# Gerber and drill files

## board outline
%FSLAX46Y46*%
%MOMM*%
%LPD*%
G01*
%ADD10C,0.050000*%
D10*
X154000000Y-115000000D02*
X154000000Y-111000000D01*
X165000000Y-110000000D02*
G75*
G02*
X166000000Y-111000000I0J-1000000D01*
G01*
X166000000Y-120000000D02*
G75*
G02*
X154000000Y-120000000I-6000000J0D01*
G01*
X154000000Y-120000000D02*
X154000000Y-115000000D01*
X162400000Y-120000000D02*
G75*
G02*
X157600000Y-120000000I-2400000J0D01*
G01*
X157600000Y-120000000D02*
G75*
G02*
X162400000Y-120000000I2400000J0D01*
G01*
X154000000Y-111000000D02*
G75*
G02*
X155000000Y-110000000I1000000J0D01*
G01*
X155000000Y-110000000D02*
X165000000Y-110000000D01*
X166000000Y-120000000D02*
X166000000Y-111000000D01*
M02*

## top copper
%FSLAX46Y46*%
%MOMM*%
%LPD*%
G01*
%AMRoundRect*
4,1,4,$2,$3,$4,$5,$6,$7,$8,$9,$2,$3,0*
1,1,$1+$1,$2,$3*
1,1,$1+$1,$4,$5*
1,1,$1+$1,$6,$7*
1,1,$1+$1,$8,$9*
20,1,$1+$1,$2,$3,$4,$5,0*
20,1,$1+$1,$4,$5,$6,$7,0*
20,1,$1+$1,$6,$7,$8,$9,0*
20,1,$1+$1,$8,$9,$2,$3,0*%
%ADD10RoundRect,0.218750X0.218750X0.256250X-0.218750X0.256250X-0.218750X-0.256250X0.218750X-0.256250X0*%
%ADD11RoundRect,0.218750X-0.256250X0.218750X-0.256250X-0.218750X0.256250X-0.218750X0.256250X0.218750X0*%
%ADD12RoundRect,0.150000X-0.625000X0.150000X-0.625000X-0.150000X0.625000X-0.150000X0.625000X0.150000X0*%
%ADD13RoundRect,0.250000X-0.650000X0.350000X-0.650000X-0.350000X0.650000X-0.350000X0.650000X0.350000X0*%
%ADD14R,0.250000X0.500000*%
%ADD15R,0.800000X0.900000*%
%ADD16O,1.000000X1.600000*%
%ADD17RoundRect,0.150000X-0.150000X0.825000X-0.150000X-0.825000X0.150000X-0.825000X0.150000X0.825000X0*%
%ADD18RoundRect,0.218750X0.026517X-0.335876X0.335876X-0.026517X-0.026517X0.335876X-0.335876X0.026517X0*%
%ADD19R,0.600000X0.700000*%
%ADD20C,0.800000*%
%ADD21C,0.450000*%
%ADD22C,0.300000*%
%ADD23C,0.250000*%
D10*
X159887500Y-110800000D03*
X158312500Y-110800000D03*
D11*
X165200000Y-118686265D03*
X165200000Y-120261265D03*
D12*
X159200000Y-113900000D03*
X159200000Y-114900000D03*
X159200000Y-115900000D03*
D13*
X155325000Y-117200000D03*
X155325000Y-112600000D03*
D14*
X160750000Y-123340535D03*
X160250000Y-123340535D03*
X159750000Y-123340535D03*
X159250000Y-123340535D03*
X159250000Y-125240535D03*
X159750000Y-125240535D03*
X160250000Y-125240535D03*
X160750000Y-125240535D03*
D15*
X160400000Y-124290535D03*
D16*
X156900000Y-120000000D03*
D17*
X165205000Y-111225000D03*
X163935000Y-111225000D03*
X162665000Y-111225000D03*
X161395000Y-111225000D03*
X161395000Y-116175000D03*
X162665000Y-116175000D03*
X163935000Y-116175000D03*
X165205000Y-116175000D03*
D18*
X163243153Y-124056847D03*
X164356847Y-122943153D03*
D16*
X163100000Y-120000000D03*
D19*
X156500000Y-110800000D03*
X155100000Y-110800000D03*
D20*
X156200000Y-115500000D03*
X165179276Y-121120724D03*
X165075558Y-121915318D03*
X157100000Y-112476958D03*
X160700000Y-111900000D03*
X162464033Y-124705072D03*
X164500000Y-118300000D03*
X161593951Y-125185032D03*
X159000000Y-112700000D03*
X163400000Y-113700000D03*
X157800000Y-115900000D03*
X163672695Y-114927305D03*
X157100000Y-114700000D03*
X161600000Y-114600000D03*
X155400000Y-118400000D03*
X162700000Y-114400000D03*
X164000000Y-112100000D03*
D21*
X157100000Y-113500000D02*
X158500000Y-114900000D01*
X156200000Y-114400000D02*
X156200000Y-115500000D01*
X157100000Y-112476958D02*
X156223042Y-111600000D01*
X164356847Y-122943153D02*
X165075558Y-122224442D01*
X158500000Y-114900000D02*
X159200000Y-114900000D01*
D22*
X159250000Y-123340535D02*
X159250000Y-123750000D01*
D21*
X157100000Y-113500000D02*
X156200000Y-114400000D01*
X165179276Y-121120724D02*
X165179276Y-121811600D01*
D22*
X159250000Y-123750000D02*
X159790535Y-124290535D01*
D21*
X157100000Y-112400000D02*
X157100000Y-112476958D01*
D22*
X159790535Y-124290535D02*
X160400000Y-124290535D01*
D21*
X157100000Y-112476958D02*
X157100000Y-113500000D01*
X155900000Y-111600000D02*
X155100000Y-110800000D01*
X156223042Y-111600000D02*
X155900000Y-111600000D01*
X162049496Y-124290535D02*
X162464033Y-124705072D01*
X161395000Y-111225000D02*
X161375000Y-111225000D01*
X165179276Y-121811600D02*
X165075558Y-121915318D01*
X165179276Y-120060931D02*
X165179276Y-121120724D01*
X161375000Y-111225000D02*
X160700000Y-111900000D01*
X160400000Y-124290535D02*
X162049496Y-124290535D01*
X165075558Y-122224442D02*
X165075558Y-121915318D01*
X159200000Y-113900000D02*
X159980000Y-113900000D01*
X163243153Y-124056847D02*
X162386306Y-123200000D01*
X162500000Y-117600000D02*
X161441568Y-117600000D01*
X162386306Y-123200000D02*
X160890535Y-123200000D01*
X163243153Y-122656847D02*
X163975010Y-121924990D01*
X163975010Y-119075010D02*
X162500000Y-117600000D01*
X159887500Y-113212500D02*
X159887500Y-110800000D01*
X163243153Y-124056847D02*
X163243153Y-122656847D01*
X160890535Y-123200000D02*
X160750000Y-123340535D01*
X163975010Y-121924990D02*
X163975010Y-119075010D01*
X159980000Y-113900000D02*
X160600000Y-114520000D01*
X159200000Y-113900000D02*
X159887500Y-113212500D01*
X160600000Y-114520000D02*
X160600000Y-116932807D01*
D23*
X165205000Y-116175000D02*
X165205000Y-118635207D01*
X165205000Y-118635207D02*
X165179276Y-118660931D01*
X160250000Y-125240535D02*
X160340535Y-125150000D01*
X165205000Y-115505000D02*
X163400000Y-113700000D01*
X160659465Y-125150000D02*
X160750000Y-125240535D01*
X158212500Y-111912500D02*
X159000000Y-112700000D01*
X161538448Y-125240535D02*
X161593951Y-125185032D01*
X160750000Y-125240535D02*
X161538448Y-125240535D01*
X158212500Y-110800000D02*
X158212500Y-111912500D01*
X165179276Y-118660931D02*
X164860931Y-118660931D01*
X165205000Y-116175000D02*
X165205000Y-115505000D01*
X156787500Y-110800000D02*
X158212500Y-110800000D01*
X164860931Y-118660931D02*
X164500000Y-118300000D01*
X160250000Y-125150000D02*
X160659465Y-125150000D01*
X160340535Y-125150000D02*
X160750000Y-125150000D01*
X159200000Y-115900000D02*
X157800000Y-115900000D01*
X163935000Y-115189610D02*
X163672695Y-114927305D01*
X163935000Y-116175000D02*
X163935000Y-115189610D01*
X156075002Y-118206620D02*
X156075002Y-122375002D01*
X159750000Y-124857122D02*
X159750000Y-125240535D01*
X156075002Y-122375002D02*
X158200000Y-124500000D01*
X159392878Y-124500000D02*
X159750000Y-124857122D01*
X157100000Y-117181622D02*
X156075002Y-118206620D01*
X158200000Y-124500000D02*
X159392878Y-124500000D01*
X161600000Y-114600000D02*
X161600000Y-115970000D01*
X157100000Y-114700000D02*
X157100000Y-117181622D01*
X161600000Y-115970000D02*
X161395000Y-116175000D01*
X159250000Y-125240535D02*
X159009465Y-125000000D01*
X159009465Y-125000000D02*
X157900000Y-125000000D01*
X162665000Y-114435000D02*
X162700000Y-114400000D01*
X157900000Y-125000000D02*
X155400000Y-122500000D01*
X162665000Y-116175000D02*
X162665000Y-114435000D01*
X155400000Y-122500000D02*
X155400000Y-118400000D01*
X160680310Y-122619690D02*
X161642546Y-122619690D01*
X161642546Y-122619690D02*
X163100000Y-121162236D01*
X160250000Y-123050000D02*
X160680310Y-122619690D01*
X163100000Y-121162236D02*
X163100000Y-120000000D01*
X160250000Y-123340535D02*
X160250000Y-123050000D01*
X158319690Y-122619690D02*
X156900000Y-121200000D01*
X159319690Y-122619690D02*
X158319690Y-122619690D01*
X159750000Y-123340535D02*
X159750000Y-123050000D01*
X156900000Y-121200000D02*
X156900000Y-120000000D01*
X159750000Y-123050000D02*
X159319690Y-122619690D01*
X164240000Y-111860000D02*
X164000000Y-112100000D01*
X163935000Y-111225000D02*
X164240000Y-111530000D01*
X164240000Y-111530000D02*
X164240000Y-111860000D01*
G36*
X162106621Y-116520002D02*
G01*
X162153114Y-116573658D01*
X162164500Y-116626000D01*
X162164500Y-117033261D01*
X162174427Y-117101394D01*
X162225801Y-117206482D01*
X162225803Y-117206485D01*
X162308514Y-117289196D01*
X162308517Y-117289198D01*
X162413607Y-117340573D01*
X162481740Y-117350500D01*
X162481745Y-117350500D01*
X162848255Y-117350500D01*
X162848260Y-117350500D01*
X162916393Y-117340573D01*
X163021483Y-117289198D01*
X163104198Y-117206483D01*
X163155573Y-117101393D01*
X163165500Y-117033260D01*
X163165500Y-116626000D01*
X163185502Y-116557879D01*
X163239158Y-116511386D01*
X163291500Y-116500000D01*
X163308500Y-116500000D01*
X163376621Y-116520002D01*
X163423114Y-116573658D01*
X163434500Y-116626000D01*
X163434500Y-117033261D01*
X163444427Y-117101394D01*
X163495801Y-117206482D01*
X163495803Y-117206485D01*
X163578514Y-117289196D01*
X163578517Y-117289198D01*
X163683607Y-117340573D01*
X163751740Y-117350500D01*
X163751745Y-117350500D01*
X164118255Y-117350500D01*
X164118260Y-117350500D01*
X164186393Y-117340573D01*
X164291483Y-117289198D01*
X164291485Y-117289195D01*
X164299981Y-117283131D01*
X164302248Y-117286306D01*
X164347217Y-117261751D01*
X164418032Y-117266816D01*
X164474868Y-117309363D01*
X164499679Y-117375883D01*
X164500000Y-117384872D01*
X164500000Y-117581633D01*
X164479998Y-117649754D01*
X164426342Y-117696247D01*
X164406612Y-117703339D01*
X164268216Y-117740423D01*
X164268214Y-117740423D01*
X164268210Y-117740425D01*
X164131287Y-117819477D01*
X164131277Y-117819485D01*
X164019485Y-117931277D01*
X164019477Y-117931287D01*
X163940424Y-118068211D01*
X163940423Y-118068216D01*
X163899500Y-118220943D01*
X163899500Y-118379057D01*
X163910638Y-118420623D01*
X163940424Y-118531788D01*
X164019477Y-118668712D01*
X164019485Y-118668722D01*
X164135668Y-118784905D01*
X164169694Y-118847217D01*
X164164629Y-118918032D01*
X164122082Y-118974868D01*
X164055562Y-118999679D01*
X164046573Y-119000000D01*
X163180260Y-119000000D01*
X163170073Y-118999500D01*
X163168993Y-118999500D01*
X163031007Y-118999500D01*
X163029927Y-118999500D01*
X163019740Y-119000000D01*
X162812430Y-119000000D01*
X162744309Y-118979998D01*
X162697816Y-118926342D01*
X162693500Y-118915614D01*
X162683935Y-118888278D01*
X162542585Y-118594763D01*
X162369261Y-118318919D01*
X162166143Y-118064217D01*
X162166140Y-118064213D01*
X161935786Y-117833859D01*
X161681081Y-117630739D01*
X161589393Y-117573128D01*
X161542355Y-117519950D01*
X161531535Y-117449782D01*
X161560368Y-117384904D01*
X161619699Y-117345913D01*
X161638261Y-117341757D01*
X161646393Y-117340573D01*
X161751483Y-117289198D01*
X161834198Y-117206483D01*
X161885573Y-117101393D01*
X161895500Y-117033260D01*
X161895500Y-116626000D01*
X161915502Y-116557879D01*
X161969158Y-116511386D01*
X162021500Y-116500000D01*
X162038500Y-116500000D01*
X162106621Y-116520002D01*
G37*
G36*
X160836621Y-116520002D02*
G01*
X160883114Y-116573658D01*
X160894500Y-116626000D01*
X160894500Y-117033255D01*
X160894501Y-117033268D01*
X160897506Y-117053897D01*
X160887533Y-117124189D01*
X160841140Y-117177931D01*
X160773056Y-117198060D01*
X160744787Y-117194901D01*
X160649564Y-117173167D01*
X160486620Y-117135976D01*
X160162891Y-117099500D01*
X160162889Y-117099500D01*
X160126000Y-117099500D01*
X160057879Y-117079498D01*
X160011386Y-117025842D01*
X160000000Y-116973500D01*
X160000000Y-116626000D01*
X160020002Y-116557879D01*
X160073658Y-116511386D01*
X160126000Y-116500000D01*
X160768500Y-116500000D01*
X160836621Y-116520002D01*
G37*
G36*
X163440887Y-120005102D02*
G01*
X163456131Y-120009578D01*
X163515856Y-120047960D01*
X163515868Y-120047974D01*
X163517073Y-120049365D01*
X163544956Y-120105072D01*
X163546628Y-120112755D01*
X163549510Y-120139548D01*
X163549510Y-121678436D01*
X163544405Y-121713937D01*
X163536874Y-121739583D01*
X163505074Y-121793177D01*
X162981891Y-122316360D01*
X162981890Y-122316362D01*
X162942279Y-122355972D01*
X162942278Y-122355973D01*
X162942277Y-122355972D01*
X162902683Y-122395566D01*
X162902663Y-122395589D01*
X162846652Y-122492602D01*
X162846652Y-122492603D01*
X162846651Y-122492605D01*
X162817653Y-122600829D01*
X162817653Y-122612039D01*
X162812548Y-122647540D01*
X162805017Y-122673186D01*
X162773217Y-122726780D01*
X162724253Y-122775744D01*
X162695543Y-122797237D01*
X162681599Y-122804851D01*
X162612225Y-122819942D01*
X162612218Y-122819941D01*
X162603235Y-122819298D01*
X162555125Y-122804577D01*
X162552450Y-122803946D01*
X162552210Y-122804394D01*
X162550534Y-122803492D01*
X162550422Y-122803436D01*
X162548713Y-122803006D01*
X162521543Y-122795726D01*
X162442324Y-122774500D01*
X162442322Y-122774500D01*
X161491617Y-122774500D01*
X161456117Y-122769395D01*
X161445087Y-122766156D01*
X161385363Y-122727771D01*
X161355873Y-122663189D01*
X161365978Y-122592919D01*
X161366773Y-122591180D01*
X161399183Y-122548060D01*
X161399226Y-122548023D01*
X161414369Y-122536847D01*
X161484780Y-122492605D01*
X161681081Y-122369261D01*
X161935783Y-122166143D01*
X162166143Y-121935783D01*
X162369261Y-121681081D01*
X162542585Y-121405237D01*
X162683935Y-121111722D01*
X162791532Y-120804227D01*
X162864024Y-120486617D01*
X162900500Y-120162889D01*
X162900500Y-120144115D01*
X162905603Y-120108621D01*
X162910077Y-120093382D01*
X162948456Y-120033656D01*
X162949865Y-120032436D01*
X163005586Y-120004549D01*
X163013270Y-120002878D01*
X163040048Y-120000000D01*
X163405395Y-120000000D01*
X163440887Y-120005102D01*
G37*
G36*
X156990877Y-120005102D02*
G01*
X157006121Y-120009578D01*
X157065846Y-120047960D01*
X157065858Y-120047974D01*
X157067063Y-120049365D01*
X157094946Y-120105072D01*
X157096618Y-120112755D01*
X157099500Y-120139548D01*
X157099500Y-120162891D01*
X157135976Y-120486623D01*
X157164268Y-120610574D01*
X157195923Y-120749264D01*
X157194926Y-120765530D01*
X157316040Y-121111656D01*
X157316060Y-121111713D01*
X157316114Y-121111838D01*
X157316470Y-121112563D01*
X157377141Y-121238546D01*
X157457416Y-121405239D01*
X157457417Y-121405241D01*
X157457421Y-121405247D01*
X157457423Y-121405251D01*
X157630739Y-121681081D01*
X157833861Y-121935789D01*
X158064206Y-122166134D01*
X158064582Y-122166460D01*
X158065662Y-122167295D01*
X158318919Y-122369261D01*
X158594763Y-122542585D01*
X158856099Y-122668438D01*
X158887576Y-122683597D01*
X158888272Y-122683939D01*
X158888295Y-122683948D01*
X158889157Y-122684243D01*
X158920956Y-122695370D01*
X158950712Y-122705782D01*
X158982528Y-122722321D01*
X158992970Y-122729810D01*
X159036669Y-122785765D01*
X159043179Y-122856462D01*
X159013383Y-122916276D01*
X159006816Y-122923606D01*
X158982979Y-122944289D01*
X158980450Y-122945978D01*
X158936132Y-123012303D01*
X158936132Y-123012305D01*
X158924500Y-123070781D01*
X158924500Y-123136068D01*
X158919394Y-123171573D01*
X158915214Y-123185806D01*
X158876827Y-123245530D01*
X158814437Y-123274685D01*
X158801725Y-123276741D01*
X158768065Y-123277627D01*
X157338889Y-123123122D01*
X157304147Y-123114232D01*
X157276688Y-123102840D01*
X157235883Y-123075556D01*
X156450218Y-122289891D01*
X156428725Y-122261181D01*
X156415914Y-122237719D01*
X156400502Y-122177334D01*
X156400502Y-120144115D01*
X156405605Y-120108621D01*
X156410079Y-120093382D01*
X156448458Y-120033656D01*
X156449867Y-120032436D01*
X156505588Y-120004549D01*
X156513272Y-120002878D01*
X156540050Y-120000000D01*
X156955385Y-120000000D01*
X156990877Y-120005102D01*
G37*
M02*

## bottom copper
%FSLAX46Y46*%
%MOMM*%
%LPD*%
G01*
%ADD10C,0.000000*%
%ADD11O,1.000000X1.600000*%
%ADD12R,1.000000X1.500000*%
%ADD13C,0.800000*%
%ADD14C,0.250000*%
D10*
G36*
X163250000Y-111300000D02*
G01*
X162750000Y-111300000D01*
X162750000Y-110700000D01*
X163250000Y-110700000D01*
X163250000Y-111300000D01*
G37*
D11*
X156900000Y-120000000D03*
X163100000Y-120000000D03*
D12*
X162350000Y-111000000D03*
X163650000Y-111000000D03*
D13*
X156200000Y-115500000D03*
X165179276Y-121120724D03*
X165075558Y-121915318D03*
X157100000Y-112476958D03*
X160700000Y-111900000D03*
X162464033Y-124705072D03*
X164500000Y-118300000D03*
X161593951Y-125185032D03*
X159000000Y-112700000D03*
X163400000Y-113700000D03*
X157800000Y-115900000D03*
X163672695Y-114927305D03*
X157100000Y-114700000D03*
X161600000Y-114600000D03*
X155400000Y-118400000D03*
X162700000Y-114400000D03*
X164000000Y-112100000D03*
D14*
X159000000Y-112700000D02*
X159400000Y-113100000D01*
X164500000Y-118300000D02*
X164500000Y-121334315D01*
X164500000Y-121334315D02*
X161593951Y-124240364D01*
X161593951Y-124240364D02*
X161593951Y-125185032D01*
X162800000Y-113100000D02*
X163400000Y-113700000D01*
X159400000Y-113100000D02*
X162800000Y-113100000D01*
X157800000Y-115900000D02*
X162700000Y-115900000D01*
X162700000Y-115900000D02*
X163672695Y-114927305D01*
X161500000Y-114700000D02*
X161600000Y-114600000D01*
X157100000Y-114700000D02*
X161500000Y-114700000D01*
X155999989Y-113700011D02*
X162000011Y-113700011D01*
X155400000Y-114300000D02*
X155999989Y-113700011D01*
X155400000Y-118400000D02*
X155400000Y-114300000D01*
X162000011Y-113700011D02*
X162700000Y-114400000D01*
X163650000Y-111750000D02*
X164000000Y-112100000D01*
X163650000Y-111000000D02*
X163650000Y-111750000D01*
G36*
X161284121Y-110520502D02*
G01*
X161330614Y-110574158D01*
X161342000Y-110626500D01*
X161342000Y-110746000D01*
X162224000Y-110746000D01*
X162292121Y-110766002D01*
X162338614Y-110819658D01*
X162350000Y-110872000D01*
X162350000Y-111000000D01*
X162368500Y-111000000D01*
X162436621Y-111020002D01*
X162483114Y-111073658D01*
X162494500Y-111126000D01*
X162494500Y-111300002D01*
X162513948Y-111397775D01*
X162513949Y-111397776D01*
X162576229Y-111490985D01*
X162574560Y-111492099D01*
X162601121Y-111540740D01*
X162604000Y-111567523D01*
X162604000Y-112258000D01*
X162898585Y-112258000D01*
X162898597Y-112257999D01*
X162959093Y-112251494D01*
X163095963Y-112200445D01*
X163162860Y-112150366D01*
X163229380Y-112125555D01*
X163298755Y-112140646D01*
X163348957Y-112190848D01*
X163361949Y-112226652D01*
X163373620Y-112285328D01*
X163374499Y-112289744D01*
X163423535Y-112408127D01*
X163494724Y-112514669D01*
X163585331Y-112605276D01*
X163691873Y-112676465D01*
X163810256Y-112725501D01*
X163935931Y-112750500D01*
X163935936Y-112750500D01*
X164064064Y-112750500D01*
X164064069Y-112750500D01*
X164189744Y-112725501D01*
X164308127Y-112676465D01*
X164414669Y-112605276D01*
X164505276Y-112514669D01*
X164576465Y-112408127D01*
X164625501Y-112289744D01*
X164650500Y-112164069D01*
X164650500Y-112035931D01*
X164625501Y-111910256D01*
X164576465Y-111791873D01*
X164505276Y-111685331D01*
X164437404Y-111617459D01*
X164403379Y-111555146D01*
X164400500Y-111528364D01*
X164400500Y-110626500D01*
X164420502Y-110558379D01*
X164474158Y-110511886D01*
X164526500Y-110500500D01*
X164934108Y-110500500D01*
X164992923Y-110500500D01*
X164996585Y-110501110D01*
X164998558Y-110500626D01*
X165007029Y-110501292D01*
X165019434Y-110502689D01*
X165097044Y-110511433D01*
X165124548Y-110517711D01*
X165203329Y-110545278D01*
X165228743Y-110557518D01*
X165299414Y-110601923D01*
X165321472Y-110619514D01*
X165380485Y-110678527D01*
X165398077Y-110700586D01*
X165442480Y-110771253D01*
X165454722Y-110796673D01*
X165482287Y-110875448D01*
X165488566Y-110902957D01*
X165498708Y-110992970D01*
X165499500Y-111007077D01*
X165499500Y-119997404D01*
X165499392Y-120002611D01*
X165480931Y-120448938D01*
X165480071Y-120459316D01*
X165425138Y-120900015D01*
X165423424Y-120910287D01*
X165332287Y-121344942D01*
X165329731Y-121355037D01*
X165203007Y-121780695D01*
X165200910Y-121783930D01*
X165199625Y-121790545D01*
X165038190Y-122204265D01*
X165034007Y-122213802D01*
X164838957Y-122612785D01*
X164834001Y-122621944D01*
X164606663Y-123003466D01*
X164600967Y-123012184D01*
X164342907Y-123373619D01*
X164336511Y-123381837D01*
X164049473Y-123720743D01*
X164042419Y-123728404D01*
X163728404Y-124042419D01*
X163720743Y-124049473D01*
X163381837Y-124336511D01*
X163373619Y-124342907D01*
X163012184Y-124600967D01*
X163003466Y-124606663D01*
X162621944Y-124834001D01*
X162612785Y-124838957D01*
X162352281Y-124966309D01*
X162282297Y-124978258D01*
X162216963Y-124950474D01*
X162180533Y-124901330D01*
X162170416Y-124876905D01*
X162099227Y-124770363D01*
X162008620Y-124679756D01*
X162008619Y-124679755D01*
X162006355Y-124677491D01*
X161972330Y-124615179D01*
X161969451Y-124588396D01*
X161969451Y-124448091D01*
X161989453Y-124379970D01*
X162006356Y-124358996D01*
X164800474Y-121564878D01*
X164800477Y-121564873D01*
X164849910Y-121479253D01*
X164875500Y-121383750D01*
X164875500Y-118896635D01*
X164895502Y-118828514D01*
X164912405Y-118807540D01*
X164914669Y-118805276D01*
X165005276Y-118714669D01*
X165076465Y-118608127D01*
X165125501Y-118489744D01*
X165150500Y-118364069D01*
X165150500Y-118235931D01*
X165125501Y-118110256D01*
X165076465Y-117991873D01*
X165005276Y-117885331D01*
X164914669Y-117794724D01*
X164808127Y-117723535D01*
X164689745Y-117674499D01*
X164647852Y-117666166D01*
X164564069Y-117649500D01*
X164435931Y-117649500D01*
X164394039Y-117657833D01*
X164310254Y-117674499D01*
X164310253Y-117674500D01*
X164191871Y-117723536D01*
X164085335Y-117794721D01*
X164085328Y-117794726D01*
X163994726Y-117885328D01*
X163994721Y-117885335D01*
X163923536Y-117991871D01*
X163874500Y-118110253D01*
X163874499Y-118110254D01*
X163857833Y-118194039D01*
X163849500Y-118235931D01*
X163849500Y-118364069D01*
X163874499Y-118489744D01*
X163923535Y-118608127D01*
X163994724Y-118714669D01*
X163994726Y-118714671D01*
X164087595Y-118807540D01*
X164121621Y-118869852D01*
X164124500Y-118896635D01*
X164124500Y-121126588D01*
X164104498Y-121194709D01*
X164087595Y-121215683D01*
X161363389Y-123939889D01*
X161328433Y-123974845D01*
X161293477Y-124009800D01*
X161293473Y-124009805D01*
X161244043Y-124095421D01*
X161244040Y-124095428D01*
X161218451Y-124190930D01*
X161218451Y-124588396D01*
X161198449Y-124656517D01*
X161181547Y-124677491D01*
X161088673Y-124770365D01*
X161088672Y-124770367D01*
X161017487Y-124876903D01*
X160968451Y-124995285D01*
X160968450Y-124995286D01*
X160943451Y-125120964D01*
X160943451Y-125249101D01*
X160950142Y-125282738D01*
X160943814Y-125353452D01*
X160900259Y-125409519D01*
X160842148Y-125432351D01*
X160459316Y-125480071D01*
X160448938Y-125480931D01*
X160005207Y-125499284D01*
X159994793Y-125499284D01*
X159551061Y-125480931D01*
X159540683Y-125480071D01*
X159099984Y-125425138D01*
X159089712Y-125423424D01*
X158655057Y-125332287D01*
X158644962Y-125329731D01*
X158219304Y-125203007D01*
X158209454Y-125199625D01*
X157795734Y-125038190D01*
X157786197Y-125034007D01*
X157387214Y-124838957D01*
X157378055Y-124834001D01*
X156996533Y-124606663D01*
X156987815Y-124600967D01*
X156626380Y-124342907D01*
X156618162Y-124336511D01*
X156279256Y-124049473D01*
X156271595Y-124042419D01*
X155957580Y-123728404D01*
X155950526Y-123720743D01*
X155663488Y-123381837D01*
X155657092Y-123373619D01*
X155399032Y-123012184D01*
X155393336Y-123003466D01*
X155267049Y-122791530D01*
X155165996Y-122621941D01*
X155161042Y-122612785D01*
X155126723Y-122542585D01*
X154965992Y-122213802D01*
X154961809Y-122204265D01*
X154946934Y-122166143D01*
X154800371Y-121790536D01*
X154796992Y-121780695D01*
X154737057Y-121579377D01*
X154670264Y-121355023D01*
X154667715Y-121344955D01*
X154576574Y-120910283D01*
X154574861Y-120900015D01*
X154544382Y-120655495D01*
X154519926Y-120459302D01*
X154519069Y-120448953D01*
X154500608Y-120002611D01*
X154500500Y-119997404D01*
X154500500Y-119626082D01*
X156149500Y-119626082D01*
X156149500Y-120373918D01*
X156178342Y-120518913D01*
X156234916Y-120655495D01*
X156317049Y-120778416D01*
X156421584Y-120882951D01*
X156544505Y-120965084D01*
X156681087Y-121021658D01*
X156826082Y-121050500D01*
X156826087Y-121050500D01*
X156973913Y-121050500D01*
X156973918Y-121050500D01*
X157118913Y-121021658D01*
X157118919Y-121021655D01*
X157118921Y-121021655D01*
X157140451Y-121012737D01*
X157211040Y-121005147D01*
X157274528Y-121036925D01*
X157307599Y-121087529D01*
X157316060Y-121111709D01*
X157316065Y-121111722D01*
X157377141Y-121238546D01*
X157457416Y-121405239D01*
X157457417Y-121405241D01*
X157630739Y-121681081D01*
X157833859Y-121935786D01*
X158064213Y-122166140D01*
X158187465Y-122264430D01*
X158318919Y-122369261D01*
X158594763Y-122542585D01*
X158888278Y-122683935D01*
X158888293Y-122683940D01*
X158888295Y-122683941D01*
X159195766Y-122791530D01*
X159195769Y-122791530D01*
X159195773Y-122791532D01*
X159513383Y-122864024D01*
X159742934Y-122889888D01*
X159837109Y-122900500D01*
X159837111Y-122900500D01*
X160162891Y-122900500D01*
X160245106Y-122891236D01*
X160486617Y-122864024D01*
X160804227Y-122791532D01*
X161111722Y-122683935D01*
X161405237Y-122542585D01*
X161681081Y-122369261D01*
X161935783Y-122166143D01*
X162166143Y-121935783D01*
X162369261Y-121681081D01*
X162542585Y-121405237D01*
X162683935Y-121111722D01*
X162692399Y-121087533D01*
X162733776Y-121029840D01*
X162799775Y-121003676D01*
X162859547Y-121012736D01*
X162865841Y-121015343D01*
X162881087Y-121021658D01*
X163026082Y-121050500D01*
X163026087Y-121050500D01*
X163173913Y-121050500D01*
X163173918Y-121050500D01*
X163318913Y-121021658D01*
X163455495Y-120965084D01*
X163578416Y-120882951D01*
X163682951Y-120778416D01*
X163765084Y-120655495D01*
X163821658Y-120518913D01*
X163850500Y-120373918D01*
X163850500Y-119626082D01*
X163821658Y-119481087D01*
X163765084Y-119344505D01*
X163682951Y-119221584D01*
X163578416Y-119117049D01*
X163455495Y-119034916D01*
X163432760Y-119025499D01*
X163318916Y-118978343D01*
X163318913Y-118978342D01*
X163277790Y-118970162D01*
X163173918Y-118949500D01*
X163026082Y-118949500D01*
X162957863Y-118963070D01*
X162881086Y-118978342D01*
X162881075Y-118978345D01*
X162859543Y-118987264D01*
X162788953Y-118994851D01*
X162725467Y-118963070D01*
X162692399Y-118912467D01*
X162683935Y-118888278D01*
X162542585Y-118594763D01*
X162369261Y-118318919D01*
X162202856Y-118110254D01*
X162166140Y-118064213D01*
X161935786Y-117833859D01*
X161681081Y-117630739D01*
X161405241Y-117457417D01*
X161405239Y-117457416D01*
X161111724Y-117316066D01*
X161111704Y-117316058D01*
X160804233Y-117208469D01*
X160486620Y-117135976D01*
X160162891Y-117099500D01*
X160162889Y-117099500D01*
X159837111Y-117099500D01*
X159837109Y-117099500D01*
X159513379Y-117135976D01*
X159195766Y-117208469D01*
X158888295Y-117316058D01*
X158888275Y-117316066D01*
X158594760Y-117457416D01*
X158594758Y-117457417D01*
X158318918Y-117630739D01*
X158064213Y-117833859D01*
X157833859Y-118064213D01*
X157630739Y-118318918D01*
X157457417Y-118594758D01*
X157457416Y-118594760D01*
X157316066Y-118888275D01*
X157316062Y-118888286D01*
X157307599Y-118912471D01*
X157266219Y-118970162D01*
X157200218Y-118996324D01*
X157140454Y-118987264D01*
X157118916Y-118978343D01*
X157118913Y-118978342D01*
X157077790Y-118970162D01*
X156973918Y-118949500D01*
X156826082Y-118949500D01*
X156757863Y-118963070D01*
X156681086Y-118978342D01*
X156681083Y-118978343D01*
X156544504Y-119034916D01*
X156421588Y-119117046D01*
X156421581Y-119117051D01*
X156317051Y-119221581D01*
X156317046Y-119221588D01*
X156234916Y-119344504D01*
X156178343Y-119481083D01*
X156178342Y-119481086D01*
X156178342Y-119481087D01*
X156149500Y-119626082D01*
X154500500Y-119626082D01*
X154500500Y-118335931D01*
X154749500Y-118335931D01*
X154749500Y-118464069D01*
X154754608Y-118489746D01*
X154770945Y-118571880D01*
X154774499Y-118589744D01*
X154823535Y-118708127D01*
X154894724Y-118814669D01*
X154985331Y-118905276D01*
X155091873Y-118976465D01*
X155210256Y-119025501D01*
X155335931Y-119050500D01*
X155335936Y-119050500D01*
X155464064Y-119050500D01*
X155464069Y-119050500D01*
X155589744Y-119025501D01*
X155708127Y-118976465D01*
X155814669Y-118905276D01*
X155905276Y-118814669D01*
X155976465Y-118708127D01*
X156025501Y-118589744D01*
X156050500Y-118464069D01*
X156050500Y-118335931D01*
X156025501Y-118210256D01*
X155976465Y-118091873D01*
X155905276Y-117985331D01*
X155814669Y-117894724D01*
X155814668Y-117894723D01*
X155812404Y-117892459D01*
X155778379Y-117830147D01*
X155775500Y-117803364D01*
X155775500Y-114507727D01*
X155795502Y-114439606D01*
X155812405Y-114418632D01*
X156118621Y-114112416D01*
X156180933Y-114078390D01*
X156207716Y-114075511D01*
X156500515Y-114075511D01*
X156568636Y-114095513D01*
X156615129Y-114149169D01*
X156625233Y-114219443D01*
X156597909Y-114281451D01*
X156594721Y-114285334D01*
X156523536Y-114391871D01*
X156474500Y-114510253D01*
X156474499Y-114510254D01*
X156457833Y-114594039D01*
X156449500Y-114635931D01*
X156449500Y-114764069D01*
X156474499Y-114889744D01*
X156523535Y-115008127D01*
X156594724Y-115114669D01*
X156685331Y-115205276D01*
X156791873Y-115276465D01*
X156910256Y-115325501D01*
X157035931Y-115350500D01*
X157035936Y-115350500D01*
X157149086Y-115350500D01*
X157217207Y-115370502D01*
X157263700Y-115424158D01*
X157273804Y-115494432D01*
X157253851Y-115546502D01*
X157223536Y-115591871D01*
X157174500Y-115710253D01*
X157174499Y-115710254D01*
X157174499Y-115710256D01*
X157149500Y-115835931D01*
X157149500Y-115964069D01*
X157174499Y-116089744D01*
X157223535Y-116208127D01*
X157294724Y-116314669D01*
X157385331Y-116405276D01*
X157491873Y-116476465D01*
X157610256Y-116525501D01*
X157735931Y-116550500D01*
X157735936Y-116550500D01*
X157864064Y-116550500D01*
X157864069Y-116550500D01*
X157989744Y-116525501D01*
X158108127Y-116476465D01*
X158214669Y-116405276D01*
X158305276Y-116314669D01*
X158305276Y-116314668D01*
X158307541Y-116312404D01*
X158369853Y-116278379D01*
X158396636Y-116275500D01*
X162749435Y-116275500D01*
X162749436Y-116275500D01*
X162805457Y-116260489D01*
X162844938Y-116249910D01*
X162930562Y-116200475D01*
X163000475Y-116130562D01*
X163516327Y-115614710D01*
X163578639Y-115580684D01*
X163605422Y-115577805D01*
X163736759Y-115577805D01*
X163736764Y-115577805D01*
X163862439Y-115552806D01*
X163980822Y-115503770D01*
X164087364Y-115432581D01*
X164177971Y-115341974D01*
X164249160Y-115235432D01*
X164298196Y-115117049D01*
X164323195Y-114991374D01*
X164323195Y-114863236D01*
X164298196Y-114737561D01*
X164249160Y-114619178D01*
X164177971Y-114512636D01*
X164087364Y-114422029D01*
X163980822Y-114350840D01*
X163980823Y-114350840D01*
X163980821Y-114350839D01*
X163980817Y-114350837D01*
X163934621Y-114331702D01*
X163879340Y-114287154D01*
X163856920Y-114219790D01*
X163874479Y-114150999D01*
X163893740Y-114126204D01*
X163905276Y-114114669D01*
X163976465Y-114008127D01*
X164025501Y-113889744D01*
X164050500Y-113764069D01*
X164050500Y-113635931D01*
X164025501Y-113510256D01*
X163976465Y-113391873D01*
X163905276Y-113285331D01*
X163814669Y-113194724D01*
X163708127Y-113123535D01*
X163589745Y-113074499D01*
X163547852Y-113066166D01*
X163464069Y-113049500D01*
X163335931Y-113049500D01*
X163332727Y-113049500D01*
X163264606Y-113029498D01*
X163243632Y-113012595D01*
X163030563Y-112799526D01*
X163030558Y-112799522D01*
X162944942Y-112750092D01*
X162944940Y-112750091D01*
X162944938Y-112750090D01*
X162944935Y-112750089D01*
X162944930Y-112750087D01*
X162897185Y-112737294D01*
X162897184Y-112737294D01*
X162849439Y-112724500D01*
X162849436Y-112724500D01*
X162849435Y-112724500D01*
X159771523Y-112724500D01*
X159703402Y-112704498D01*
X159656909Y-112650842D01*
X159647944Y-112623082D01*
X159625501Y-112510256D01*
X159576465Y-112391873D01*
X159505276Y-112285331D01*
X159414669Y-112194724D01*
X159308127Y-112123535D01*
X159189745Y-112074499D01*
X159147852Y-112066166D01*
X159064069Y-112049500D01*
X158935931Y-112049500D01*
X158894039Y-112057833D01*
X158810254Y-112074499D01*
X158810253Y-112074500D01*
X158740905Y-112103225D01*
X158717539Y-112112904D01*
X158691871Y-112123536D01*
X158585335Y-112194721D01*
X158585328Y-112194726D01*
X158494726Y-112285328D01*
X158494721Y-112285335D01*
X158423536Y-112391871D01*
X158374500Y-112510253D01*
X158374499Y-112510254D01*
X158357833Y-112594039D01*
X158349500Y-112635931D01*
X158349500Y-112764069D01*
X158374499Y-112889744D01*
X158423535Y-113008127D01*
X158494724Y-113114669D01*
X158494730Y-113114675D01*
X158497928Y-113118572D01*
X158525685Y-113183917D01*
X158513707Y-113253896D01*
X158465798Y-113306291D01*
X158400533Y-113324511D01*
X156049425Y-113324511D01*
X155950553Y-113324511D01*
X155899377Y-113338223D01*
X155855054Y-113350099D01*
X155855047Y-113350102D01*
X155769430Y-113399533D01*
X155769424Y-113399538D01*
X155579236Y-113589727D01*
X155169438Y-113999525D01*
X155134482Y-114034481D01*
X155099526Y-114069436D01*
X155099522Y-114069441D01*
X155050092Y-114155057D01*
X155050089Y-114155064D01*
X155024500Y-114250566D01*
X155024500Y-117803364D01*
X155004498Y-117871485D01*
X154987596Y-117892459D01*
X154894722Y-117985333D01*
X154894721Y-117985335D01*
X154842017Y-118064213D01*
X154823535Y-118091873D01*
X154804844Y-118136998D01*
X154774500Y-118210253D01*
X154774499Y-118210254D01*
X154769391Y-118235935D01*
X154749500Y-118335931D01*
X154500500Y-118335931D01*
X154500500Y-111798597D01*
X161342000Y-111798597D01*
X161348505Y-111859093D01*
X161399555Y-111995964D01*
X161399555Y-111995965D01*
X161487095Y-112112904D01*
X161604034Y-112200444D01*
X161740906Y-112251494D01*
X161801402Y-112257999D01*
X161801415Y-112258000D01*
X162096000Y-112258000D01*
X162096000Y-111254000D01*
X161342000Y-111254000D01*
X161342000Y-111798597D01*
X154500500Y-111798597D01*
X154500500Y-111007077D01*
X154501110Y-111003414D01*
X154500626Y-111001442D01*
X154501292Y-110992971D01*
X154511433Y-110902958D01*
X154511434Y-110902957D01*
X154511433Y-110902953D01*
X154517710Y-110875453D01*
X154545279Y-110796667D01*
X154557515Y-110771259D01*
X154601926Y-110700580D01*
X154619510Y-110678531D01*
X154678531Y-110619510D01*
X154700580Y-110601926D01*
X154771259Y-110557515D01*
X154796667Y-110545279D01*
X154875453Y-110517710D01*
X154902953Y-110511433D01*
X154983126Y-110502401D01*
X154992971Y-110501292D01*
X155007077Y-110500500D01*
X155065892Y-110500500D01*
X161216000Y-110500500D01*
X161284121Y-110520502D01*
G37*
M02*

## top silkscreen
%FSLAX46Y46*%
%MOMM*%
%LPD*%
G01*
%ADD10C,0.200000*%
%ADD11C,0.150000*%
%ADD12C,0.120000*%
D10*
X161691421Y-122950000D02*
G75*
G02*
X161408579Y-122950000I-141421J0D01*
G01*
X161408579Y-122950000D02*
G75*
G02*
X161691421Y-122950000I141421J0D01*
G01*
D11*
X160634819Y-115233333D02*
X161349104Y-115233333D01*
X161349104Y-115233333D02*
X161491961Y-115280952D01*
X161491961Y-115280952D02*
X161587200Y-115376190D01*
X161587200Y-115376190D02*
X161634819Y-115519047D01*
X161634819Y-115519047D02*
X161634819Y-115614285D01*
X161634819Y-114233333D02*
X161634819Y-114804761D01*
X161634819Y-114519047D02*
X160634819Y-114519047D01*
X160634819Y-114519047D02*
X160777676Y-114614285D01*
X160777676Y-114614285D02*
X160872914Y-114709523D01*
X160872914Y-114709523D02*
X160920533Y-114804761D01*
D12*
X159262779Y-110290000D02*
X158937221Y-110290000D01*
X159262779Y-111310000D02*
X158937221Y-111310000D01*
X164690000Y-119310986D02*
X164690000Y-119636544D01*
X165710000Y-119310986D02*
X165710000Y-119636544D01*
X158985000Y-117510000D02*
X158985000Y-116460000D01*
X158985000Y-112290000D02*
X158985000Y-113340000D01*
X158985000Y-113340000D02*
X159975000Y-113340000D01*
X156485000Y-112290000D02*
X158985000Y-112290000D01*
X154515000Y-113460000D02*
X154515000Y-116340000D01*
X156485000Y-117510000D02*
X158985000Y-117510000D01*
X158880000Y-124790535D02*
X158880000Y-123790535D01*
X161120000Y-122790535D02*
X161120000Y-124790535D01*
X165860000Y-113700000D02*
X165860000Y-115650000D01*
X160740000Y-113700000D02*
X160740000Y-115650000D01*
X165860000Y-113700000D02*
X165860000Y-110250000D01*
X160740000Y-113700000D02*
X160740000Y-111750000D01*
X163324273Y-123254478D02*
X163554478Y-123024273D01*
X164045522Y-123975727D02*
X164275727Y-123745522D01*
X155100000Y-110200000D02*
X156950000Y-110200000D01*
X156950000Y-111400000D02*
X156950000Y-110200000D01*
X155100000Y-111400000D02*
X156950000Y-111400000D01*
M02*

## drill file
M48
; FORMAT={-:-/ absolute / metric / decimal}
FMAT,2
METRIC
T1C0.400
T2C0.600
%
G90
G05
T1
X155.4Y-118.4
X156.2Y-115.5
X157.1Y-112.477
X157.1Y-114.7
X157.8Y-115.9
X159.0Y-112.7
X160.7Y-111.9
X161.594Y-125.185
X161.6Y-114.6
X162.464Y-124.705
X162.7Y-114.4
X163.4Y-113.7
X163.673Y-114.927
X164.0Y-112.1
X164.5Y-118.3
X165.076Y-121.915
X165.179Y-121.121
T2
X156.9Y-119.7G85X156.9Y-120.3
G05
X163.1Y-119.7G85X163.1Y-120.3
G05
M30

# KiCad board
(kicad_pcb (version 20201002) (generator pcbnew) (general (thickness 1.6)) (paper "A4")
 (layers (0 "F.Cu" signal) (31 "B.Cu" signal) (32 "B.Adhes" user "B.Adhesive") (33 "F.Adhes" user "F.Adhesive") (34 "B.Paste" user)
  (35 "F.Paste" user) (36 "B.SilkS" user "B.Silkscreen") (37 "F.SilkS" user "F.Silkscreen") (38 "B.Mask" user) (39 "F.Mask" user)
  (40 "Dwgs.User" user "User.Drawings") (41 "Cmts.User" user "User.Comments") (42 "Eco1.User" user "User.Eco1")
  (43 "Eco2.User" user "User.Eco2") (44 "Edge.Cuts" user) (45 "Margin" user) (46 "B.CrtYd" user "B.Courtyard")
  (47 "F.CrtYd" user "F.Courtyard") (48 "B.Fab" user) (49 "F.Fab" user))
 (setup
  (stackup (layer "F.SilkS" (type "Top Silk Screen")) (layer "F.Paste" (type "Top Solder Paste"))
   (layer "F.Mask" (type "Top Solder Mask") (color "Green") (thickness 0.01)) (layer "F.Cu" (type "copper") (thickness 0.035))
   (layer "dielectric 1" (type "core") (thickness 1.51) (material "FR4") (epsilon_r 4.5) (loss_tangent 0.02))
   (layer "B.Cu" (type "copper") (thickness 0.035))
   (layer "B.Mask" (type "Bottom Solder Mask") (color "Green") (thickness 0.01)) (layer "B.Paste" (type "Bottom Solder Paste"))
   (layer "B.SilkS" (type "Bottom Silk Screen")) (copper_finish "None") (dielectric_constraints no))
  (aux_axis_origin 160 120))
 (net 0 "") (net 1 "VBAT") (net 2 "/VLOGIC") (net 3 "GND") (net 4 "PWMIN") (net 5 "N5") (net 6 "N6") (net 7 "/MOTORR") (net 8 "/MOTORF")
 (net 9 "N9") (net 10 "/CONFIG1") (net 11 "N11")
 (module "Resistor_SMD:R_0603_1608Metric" (layer "F.Cu") (at 159.1 110.8 180)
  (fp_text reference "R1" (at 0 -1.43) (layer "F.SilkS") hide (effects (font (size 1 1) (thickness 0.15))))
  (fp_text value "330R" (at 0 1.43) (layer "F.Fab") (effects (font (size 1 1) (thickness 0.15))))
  (fp_line (start -0.162779 0.51) (end 0.162779 0.51) (layer "F.SilkS") (width 0.12))
  (fp_line (start -0.162779 -0.51) (end 0.162779 -0.51) (layer "F.SilkS") (width 0.12))
  (pad "1" smd roundrect (at -0.7875 0 180) (size 0.875 0.95) (layers "F.Cu" "F.Paste" "F.Mask") (roundrect_rratio 0.25) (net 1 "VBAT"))
  (pad "2" smd roundrect (at 0.7875 0 180) (size 0.875 0.95) (layers "F.Cu" "F.Paste" "F.Mask") (roundrect_rratio 0.25) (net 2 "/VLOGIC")))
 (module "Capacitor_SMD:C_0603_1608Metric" (layer "F.Cu") (at 165.2 119.473765 -90)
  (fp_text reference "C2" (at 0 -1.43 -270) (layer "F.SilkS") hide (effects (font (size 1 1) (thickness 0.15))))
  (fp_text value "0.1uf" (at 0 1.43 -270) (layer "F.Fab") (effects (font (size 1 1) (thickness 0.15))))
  (fp_line (start -0.162779 0.51) (end 0.162779 0.51) (layer "F.SilkS") (width 0.12))
  (fp_line (start -0.162779 -0.51) (end 0.162779 -0.51) (layer "F.SilkS") (width 0.12))
  (pad "1" smd roundrect (at -0.7875 0 270) (size 0.875 0.95) (layers "F.Cu" "F.Paste" "F.Mask") (roundrect_rratio 0.25) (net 2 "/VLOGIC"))
  (pad "2" smd roundrect (at 0.7875 0 270) (size 0.875 0.95) (layers "F.Cu" "F.Paste" "F.Mask") (roundrect_rratio 0.25) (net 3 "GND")))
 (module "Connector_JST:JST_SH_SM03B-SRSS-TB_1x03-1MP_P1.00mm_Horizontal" (layer "F.Cu") (at 157.2 114.9 -90)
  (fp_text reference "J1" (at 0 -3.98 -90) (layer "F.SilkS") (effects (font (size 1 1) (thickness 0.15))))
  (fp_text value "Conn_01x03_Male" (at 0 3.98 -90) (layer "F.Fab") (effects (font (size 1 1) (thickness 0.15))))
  (fp_line (start 2.61 -1.785) (end 1.56 -1.785) (layer "F.SilkS") (width 0.12))
  (fp_line (start -2.61 -1.785) (end -1.56 -1.785) (layer "F.SilkS") (width 0.12))
  (fp_line (start -1.56 -1.785) (end -1.56 -2.775) (layer "F.SilkS") (width 0.12))
  (fp_line (start -2.61 0.715) (end -2.61 -1.785) (layer "F.SilkS") (width 0.12))
  (fp_line (start -1.44 2.685) (end 1.44 2.685) (layer "F.SilkS") (width 0.12))
  (fp_line (start 2.61 0.715) (end 2.61 -1.785) (layer "F.SilkS") (width 0.12))
  (pad "1" smd roundrect (at -1 -2 270) (size 0.6 1.55) (layers "F.Cu" "F.Paste" "F.Mask") (roundrect_rratio 0.25) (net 1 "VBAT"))
  (pad "2" smd roundrect (at 0 -2 270) (size 0.6 1.55) (layers "F.Cu" "F.Paste" "F.Mask") (roundrect_rratio 0.25) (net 3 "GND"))
  (pad "3" smd roundrect (at 1 -2 270) (size 0.6 1.55) (layers "F.Cu" "F.Paste" "F.Mask") (roundrect_rratio 0.25) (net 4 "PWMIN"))
  (pad "MP" smd roundrect (at 2.3 1.875 270) (size 1.2 1.8) (layers "F.Cu" "F.Paste" "F.Mask") (roundrect_rratio 0.208333))
  (pad "MP" smd roundrect (at -2.3 1.875 270) (size 1.2 1.8) (layers "F.Cu" "F.Paste" "F.Mask") (roundrect_rratio 0.208333)))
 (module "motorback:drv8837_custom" (layer "F.Cu") (at 160 124.290535 -90)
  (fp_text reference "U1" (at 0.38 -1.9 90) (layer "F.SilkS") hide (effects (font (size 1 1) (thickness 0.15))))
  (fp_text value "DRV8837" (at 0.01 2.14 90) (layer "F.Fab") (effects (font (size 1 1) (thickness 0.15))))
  (fp_line (start 0.5 1.12) (end -0.5 1.12) (layer "F.SilkS") (width 0.12))
  (fp_line (start -1.5 -1.12) (end 0.5 -1.12) (layer "F.SilkS") (width 0.12))
  (pad "" smd rect (at 0 -0.4 270) (size 0.75 0.65) (layers "F.Paste"))
  (pad "1" smd rect (at -0.95 -0.75 270) (size 0.5 0.25) (layers "F.Cu" "F.Paste" "F.Mask") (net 1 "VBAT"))
  (pad "2" smd rect (at -0.95 -0.25 270) (size 0.5 0.25) (layers "F.Cu" "F.Paste" "F.Mask") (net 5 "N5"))
  (pad "3" smd rect (at -0.95 0.25 270) (size 0.5 0.25) (layers "F.Cu" "F.Paste" "F.Mask") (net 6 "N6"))
  (pad "4" smd rect (at -0.95 0.75 270) (size 0.5 0.25) (layers "F.Cu" "F.Paste" "F.Mask") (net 3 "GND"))
  (pad "5" smd rect (at 0.95 0.75 270) (size 0.5 0.25) (layers "F.Cu" "F.Paste" "F.Mask") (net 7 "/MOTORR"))
  (pad "6" smd rect (at 0.95 0.25 270) (size 0.5 0.25) (layers "F.Cu" "F.Paste" "F.Mask") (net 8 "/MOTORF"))
  (pad "7" smd rect (at 0.95 -0.25 270) (size 0.5 0.25) (layers "F.Cu" "F.Paste" "F.Mask") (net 2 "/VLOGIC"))
  (pad "8" smd rect (at 0.95 -0.75 270) (size 0.5 0.25) (layers "F.Cu" "F.Paste" "F.Mask") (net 2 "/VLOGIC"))
  (pad "9" smd rect (at 0 -0.4 270) (size 0.9 0.8) (layers "F.Cu" "F.Mask") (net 3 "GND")))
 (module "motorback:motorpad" (layer "F.Cu") (at 156.9 120)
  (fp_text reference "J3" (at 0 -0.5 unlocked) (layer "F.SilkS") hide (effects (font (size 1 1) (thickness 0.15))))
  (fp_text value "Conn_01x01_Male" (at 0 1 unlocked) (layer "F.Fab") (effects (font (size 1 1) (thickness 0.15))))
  (pad "1" thru_hole oval (at 0 0) (size 1 1.6) (drill oval 0.6 1.2) (layers *.Cu *.Mask) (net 6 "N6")))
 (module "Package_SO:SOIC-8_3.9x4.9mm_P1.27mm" (layer "F.Cu") (at 163.3 113.7 -90)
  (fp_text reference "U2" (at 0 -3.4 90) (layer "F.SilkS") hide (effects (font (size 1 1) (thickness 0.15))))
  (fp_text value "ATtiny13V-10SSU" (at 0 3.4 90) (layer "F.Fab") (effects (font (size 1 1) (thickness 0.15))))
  (fp_line (start 0 -2.56) (end 1.95 -2.56) (layer "F.SilkS") (width 0.12))
  (fp_line (start 0 2.56) (end 1.95 2.56) (layer "F.SilkS") (width 0.12))
  (fp_line (start 0 -2.56) (end -3.45 -2.56) (layer "F.SilkS") (width 0.12))
  (fp_line (start 0 2.56) (end -1.95 2.56) (layer "F.SilkS") (width 0.12))
  (pad "1" smd roundrect (at -2.475 -1.905 270) (size 1.95 0.6) (layers "F.Cu" "F.Paste" "F.Mask") (roundrect_rratio 0.25) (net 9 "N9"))
  (pad "2" smd roundrect (at -2.475 -0.635 270) (size 1.95 0.6) (layers "F.Cu" "F.Paste" "F.Mask") (roundrect_rratio 0.25)
   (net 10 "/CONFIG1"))
  (pad "3" smd roundrect (at -2.475 0.635 270) (size 1.95 0.6) (layers "F.Cu" "F.Paste" "F.Mask") (roundrect_rratio 0.25) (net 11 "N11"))
  (pad "4" smd roundrect (at -2.475 1.905 270) (size 1.95 0.6) (layers "F.Cu" "F.Paste" "F.Mask") (roundrect_rratio 0.25) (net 3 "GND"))
  (pad "5" smd roundrect (at 2.475 1.905 270) (size 1.95 0.6) (layers "F.Cu" "F.Paste" "F.Mask") (roundrect_rratio 0.25) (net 8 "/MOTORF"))
  (pad "6" smd roundrect (at 2.475 0.635 270) (size 1.95 0.6) (layers "F.Cu" "F.Paste" "F.Mask") (roundrect_rratio 0.25) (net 7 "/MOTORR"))
  (pad "7" smd roundrect (at 2.475 -0.635 270) (size 1.95 0.6) (layers "F.Cu" "F.Paste" "F.Mask") (roundrect_rratio 0.25) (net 4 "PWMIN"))
  (pad "8" smd roundrect (at 2.475 -1.905 270) (size 1.95 0.6) (layers "F.Cu" "F.Paste" "F.Mask") (roundrect_rratio 0.25) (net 2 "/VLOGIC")))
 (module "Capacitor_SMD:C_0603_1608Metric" (layer "F.Cu") (at 163.8 123.5 45)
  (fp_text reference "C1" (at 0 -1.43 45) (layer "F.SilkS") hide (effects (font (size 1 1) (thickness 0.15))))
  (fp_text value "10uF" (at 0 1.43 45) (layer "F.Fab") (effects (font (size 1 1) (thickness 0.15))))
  (fp_line (start -0.162779 -0.51) (end 0.162779 -0.51) (layer "F.SilkS") (width 0.12))
  (fp_line (start -0.162779 0.51) (end 0.162779 0.51) (layer "F.SilkS") (width 0.12))
  (pad "1" smd roundrect (at -0.7875 0 45) (size 0.875 0.95) (layers "F.Cu" "F.Paste" "F.Mask") (roundrect_rratio 0.25) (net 1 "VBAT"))
  (pad "2" smd roundrect (at 0.7875 0 45) (size 0.875 0.95) (layers "F.Cu" "F.Paste" "F.Mask") (roundrect_rratio 0.25) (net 3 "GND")))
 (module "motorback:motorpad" (layer "F.Cu") (at 163 120)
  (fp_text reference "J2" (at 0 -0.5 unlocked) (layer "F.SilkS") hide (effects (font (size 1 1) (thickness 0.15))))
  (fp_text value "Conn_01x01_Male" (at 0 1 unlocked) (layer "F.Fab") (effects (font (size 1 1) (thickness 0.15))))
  (pad "1" thru_hole oval (at 0.1 0) (size 1 1.6) (drill oval 0.6 1.2) (layers *.Cu *.Mask) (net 5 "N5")))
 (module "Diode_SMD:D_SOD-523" (layer "F.Cu") (at 155.8 110.8 180)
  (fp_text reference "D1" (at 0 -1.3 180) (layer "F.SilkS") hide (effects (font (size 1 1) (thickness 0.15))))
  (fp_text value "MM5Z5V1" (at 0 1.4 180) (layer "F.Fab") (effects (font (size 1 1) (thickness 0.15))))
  (fp_line (start 0.7 0.6) (end -1.15 0.6) (layer "F.SilkS") (width 0.12))
  (fp_line (start -1.15 -0.6) (end -1.15 0.6) (layer "F.SilkS") (width 0.12))
  (fp_line (start 0.7 -0.6) (end -1.15 -0.6) (layer "F.SilkS") (width 0.12))
  (pad "1" smd rect (at -0.7 0) (size 0.6 0.7) (layers "F.Cu" "F.Paste" "F.Mask") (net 2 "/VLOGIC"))
  (pad "2" smd rect (at 0.7 0) (size 0.6 0.7) (layers "F.Cu" "F.Paste" "F.Mask") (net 3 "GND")))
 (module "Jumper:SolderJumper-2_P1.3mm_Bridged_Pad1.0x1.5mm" (layer "B.Cu") (at 163 111)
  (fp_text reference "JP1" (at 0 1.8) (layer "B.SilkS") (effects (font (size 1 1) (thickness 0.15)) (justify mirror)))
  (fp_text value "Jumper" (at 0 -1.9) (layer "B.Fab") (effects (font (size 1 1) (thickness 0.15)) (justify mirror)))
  (fp_poly (pts (xy -0.25 0.3) (xy 0.25 0.3) (xy 0.25 -0.3) (xy -0.25 -0.3)) (layer "B.Cu") (width 0))
  (pad "1" smd rect (at -0.65 0) (size 1 1.5) (layers "B.Cu" "B.Mask") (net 3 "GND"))
  (pad "2" smd rect (at 0.65 0) (size 1 1.5) (layers "B.Cu" "B.Mask") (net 10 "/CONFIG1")))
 (gr_circle (center 161.55 122.95) (end 161.691421 122.95) (layer "F.SilkS") (width 0.2))
 (gr_line (start 154 115) (end 154 111) (layer "Edge.Cuts") (width 0.05))
 (gr_arc (start 165 111) (end 166 111) (angle -90) (layer "Edge.Cuts") (width 0.05))
 (gr_arc (start 160 120) (end 154 120) (angle -180) (layer "Edge.Cuts") (width 0.05))
 (gr_line (start 154 120) (end 154 115) (layer "Edge.Cuts") (width 0.05))
 (gr_circle (center 160 120) (end 162.4 120) (layer "Edge.Cuts") (width 0.05))
 (gr_arc (start 155 111) (end 155 110) (angle -90) (layer "Edge.Cuts") (width 0.05))
 (gr_line (start 155 110) (end 165 110) (layer "Edge.Cuts") (width 0.05))
 (gr_line (start 166 120) (end 166 111) (layer "Edge.Cuts") (width 0.05))
 (segment (start 157.1 113.5) (end 158.5 114.9) (width 0.45) (layer "F.Cu") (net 3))
 (segment (start 156.2 114.4) (end 156.2 115.5) (width 0.45) (layer "F.Cu") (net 3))
 (segment (start 157.1 112.476958) (end 156.223042 111.6) (width 0.45) (layer "F.Cu") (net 3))
 (segment (start 164.356847 122.943153) (end 165.075558 122.224442) (width 0.45) (layer "F.Cu") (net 3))
 (segment (start 158.5 114.9) (end 159.2 114.9) (width 0.45) (layer "F.Cu") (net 3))
 (segment (start 159.25 123.340535) (end 159.25 123.75) (width 0.3) (layer "F.Cu") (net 3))
 (segment (start 157.1 113.5) (end 156.2 114.4) (width 0.45) (layer "F.Cu") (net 3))
 (segment (start 165.179276 121.120724) (end 165.179276 121.8116) (width 0.45) (layer "F.Cu") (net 3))
 (segment (start 159.25 123.75) (end 159.790535 124.290535) (width 0.3) (layer "F.Cu") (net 3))
 (segment (start 157.1 112.4) (end 157.1 112.476958) (width 0.45) (layer "F.Cu") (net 3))
 (segment (start 159.790535 124.290535) (end 160.4 124.290535) (width 0.3) (layer "F.Cu") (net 3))
 (segment (start 157.1 112.476958) (end 157.1 113.5) (width 0.45) (layer "F.Cu") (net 3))
 (segment (start 155.9 111.6) (end 155.1 110.8) (width 0.45) (layer "F.Cu") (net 3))
 (segment (start 156.223042 111.6) (end 155.9 111.6) (width 0.45) (layer "F.Cu") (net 3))
 (segment (start 162.049496 124.290535) (end 162.464033 124.705072) (width 0.45) (layer "F.Cu") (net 3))
 (segment (start 161.395 111.225) (end 161.375 111.225) (width 0.45) (layer "F.Cu") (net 3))
 (segment (start 165.179276 121.8116) (end 165.075558 121.915318) (width 0.45) (layer "F.Cu") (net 3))
 (segment (start 165.179276 120.060931) (end 165.179276 121.120724) (width 0.45) (layer "F.Cu") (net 3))
 (segment (start 161.375 111.225) (end 160.7 111.9) (width 0.45) (layer "F.Cu") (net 3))
 (segment (start 160.4 124.290535) (end 162.049496 124.290535) (width 0.45) (layer "F.Cu") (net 3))
 (segment (start 165.075558 122.224442) (end 165.075558 121.915318) (width 0.45) (layer "F.Cu") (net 3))
 (via (at 156.2 115.5) (size 0.8) (drill 0.4) (layers "F.Cu" "B.Cu") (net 3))
 (via (at 165.179276 121.120724) (size 0.8) (drill 0.4) (layers "F.Cu" "B.Cu") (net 3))
 (via (at 165.075558 121.915318) (size 0.8) (drill 0.4) (layers "F.Cu" "B.Cu") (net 3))
 (via (at 157.1 112.476958) (size 0.8) (drill 0.4) (layers "F.Cu" "B.Cu") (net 3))
 (via (at 160.7 111.9) (size 0.8) (drill 0.4) (layers "F.Cu" "B.Cu") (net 3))
 (via (at 162.464033 124.705072) (size 0.8) (drill 0.4) (layers "F.Cu" "B.Cu") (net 3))
 (segment (start 159.2 113.9) (end 159.98 113.9) (width 0.45) (layer "F.Cu") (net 1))
 (segment (start 163.243153 124.056847) (end 162.386306 123.2) (width 0.45) (layer "F.Cu") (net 1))
 (segment (start 162.5 117.6) (end 161.441568 117.6) (width 0.45) (layer "F.Cu") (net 1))
 (segment (start 162.386306 123.2) (end 160.890535 123.2) (width 0.45) (layer "F.Cu") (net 1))
 (segment (start 163.243153 122.656847) (end 163.97501 121.92499) (width 0.45) (layer "F.Cu") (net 1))
 (segment (start 163.97501 119.07501) (end 162.5 117.6) (width 0.45) (layer "F.Cu") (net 1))
 (segment (start 159.8875 113.2125) (end 159.8875 110.8) (width 0.45) (layer "F.Cu") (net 1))
 (segment (start 163.243153 124.056847) (end 163.243153 122.656847) (width 0.45) (layer "F.Cu") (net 1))
 (segment (start 160.890535 123.2) (end 160.75 123.340535) (width 0.45) (layer "F.Cu") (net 1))
 (segment (start 163.97501 121.92499) (end 163.97501 119.07501) (width 0.45) (layer "F.Cu") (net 1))
 (segment (start 159.98 113.9) (end 160.6 114.52) (width 0.45) (layer "F.Cu") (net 1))
 (segment (start 159.2 113.9) (end 159.8875 113.2125) (width 0.45) (layer "F.Cu") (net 1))
 (segment (start 160.6 114.52) (end 160.6 116.932807) (width 0.45) (layer "F.Cu") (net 1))
 (segment (start 165.205 116.175) (end 165.205 118.635207) (width 0.25) (layer "F.Cu") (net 2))
 (segment (start 165.205 118.635207) (end 165.179276 118.660931) (width 0.25) (layer "F.Cu") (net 2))
 (segment (start 160.25 125.240535) (end 160.340535 125.15) (width 0.25) (layer "F.Cu") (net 2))
 (segment (start 165.205 115.505) (end 163.4 113.7) (width 0.25) (layer "F.Cu") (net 2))
 (segment (start 160.659465 125.15) (end 160.75 125.240535) (width 0.25) (layer "F.Cu") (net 2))
 (segment (start 158.2125 111.9125) (end 159 112.7) (width 0.25) (layer "F.Cu") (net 2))
 (segment (start 161.538448 125.240535) (end 161.593951 125.185032) (width 0.25) (layer "F.Cu") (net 2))
 (segment (start 160.75 125.240535) (end 161.538448 125.240535) (width 0.25) (layer "F.Cu") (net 2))
 (segment (start 158.2125 110.8) (end 158.2125 111.9125) (width 0.25) (layer "F.Cu") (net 2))
 (segment (start 165.179276 118.660931) (end 164.860931 118.660931) (width 0.25) (layer "F.Cu") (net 2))
 (segment (start 165.205 116.175) (end 165.205 115.505) (width 0.25) (layer "F.Cu") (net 2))
 (segment (start 156.7875 110.8) (end 158.2125 110.8) (width 0.25) (layer "F.Cu") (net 2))
 (segment (start 164.860931 118.660931) (end 164.5 118.3) (width 0.25) (layer "F.Cu") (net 2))
 (segment (start 160.25 125.15) (end 160.659465 125.15) (width 0.25) (layer "F.Cu") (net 2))
 (segment (start 160.340535 125.15) (end 160.75 125.15) (width 0.25) (layer "F.Cu") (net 2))
 (via (at 164.5 118.3) (size 0.8) (drill 0.4) (layers "F.Cu" "B.Cu") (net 2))
 (via (at 161.593951 125.185032) (size 0.8) (drill 0.4) (layers "F.Cu" "B.Cu") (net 2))
 (via (at 159 112.7) (size 0.8) (drill 0.4) (layers "F.Cu" "B.Cu") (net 2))
 (via (at 163.4 113.7) (size 0.8) (drill 0.4) (layers "F.Cu" "B.Cu") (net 2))
 (segment (start 159 112.7) (end 159.4 113.1) (width 0.25) (layer "B.Cu") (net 2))
 (segment (start 164.5 118.3) (end 164.5 121.334315) (width 0.25) (layer "B.Cu") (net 2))
 (segment (start 164.5 121.334315) (end 161.593951 124.240364) (width 0.25) (layer "B.Cu") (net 2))
 (segment (start 161.593951 124.240364) (end 161.593951 125.185032) (width 0.25) (layer "B.Cu") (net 2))
 (segment (start 162.8 113.1) (end 163.4 113.7) (width 0.25) (layer "B.Cu") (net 2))
 (segment (start 159.4 113.1) (end 162.8 113.1) (width 0.25) (layer "B.Cu") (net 2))
 (segment (start 159.2 115.9) (end 157.8 115.9) (width 0.25) (layer "F.Cu") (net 4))
 (segment (start 163.935 115.18961) (end 163.672695 114.927305) (width 0.25) (layer "F.Cu") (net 4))
 (segment (start 163.935 116.175) (end 163.935 115.18961) (width 0.25) (layer "F.Cu") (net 4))
 (via (at 157.8 115.9) (size 0.8) (drill 0.4) (layers "F.Cu" "B.Cu") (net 4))
 (via (at 163.672695 114.927305) (size 0.8) (drill 0.4) (layers "F.Cu" "B.Cu") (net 4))
 (segment (start 157.8 115.9) (end 162.7 115.9) (width 0.25) (layer "B.Cu") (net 4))
 (segment (start 162.7 115.9) (end 163.672695 114.927305) (width 0.25) (layer "B.Cu") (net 4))
 (segment (start 156.075002 118.20662) (end 156.075002 122.375002) (width 0.25) (layer "F.Cu") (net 8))
 (segment (start 159.75 124.857122) (end 159.75 125.240535) (width 0.25) (layer "F.Cu") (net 8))
 (segment (start 156.075002 122.375002) (end 158.2 124.5) (width 0.25) (layer "F.Cu") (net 8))
 (segment (start 159.392878 124.5) (end 159.75 124.857122) (width 0.25) (layer "F.Cu") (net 8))
 (segment (start 157.1 117.181622) (end 156.075002 118.20662) (width 0.25) (layer "F.Cu") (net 8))
 (segment (start 158.2 124.5) (end 159.392878 124.5) (width 0.25) (layer "F.Cu") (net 8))
 (segment (start 161.6 114.6) (end 161.6 115.97) (width 0.25) (layer "F.Cu") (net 8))
 (segment (start 157.1 114.7) (end 157.1 117.181622) (width 0.25) (layer "F.Cu") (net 8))
 (segment (start 161.6 115.97) (end 161.395 116.175) (width 0.25) (layer "F.Cu") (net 8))
 (via (at 157.1 114.7) (size 0.8) (drill 0.4) (layers "F.Cu" "B.Cu") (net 8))
 (via (at 161.6 114.6) (size 0.8) (drill 0.4) (layers "F.Cu" "B.Cu") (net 8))
 (segment (start 161.5 114.7) (end 161.6 114.6) (width 0.25) (layer "B.Cu") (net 8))
 (segment (start 157.1 114.7) (end 161.5 114.7) (width 0.25) (layer "B.Cu") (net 8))
 (segment (start 159.25 125.240535) (end 159.009465 125) (width 0.25) (layer "F.Cu") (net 7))
 (segment (start 159.009465 125) (end 157.9 125) (width 0.25) (layer "F.Cu") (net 7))
 (segment (start 162.665 114.435) (end 162.7 114.4) (width 0.25) (layer "F.Cu") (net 7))
 (segment (start 157.9 125) (end 155.4 122.5) (width 0.25) (layer "F.Cu") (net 7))
 (segment (start 162.665 116.175) (end 162.665 114.435) (width 0.25) (layer "F.Cu") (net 7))
 (segment (start 155.4 122.5) (end 155.4 118.4) (width 0.25) (layer "F.Cu") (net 7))
 (via (at 155.4 118.4) (size 0.8) (drill 0.4) (layers "F.Cu" "B.Cu") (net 7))
 (via (at 162.7 114.4) (size 0.8) (drill 0.4) (layers "F.Cu" "B.Cu") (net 7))
 (segment (start 155.999989 113.700011) (end 162.000011 113.700011) (width 0.25) (layer "B.Cu") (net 7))
 (segment (start 155.4 114.3) (end 155.999989 113.700011) (width 0.25) (layer "B.Cu") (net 7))
 (segment (start 155.4 118.4) (end 155.4 114.3) (width 0.25) (layer "B.Cu") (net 7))
 (segment (start 162.000011 113.700011) (end 162.7 114.4) (width 0.25) (layer "B.Cu") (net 7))
 (segment (start 160.68031 122.61969) (end 161.642546 122.61969) (width 0.25) (layer "F.Cu") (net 5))
 (segment (start 161.642546 122.61969) (end 163.1 121.162236) (width 0.25) (layer "F.Cu") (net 5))
 (segment (start 160.25 123.05) (end 160.68031 122.61969) (width 0.25) (layer "F.Cu") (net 5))
 (segment (start 163.1 121.162236) (end 163.1 120) (width 0.25) (layer "F.Cu") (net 5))
 (segment (start 160.25 123.340535) (end 160.25 123.05) (width 0.25) (layer "F.Cu") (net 5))
 (segment (start 158.31969 122.61969) (end 156.9 121.2) (width 0.25) (layer "F.Cu") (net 6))
 (segment (start 159.31969 122.61969) (end 158.31969 122.61969) (width 0.25) (layer "F.Cu") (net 6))
 (segment (start 159.75 123.340535) (end 159.75 123.05) (width 0.25) (layer "F.Cu") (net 6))
 (segment (start 156.9 121.2) (end 156.9 120) (width 0.25) (layer "F.Cu") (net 6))
 (segment (start 159.75 123.05) (end 159.31969 122.61969) (width 0.25) (layer "F.Cu") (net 6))
 (segment (start 164.24 111.86) (end 164 112.1) (width 0.25) (layer "F.Cu") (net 10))
 (segment (start 163.935 111.225) (end 164.24 111.53) (width 0.25) (layer "F.Cu") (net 10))
 (segment (start 164.24 111.53) (end 164.24 111.86) (width 0.25) (layer "F.Cu") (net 10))
 (via (at 164 112.1) (size 0.8) (drill 0.4) (layers "F.Cu" "B.Cu") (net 10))
 (segment (start 163.65 111.75) (end 164 112.1) (width 0.25) (layer "B.Cu") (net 10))
 (segment (start 163.65 111) (end 163.65 111.75) (width 0.25) (layer "B.Cu") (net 10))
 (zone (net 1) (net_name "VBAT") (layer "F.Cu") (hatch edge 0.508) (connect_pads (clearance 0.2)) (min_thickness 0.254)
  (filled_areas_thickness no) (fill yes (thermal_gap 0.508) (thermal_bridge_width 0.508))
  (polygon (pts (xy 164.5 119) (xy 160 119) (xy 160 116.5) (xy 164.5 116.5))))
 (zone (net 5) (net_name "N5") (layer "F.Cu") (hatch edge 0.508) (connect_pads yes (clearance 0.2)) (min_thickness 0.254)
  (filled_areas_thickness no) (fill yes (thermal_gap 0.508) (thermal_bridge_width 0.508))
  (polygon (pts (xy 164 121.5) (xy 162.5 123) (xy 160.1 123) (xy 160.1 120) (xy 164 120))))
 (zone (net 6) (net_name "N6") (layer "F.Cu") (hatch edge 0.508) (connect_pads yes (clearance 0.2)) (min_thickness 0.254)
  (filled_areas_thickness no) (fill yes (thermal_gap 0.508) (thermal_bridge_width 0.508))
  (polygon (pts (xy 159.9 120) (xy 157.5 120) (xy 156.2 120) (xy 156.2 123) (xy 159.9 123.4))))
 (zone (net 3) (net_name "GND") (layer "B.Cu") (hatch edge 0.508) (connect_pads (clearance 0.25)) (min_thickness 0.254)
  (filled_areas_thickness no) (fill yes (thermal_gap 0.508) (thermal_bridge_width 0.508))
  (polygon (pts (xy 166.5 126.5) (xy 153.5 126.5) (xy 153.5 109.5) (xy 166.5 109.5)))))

